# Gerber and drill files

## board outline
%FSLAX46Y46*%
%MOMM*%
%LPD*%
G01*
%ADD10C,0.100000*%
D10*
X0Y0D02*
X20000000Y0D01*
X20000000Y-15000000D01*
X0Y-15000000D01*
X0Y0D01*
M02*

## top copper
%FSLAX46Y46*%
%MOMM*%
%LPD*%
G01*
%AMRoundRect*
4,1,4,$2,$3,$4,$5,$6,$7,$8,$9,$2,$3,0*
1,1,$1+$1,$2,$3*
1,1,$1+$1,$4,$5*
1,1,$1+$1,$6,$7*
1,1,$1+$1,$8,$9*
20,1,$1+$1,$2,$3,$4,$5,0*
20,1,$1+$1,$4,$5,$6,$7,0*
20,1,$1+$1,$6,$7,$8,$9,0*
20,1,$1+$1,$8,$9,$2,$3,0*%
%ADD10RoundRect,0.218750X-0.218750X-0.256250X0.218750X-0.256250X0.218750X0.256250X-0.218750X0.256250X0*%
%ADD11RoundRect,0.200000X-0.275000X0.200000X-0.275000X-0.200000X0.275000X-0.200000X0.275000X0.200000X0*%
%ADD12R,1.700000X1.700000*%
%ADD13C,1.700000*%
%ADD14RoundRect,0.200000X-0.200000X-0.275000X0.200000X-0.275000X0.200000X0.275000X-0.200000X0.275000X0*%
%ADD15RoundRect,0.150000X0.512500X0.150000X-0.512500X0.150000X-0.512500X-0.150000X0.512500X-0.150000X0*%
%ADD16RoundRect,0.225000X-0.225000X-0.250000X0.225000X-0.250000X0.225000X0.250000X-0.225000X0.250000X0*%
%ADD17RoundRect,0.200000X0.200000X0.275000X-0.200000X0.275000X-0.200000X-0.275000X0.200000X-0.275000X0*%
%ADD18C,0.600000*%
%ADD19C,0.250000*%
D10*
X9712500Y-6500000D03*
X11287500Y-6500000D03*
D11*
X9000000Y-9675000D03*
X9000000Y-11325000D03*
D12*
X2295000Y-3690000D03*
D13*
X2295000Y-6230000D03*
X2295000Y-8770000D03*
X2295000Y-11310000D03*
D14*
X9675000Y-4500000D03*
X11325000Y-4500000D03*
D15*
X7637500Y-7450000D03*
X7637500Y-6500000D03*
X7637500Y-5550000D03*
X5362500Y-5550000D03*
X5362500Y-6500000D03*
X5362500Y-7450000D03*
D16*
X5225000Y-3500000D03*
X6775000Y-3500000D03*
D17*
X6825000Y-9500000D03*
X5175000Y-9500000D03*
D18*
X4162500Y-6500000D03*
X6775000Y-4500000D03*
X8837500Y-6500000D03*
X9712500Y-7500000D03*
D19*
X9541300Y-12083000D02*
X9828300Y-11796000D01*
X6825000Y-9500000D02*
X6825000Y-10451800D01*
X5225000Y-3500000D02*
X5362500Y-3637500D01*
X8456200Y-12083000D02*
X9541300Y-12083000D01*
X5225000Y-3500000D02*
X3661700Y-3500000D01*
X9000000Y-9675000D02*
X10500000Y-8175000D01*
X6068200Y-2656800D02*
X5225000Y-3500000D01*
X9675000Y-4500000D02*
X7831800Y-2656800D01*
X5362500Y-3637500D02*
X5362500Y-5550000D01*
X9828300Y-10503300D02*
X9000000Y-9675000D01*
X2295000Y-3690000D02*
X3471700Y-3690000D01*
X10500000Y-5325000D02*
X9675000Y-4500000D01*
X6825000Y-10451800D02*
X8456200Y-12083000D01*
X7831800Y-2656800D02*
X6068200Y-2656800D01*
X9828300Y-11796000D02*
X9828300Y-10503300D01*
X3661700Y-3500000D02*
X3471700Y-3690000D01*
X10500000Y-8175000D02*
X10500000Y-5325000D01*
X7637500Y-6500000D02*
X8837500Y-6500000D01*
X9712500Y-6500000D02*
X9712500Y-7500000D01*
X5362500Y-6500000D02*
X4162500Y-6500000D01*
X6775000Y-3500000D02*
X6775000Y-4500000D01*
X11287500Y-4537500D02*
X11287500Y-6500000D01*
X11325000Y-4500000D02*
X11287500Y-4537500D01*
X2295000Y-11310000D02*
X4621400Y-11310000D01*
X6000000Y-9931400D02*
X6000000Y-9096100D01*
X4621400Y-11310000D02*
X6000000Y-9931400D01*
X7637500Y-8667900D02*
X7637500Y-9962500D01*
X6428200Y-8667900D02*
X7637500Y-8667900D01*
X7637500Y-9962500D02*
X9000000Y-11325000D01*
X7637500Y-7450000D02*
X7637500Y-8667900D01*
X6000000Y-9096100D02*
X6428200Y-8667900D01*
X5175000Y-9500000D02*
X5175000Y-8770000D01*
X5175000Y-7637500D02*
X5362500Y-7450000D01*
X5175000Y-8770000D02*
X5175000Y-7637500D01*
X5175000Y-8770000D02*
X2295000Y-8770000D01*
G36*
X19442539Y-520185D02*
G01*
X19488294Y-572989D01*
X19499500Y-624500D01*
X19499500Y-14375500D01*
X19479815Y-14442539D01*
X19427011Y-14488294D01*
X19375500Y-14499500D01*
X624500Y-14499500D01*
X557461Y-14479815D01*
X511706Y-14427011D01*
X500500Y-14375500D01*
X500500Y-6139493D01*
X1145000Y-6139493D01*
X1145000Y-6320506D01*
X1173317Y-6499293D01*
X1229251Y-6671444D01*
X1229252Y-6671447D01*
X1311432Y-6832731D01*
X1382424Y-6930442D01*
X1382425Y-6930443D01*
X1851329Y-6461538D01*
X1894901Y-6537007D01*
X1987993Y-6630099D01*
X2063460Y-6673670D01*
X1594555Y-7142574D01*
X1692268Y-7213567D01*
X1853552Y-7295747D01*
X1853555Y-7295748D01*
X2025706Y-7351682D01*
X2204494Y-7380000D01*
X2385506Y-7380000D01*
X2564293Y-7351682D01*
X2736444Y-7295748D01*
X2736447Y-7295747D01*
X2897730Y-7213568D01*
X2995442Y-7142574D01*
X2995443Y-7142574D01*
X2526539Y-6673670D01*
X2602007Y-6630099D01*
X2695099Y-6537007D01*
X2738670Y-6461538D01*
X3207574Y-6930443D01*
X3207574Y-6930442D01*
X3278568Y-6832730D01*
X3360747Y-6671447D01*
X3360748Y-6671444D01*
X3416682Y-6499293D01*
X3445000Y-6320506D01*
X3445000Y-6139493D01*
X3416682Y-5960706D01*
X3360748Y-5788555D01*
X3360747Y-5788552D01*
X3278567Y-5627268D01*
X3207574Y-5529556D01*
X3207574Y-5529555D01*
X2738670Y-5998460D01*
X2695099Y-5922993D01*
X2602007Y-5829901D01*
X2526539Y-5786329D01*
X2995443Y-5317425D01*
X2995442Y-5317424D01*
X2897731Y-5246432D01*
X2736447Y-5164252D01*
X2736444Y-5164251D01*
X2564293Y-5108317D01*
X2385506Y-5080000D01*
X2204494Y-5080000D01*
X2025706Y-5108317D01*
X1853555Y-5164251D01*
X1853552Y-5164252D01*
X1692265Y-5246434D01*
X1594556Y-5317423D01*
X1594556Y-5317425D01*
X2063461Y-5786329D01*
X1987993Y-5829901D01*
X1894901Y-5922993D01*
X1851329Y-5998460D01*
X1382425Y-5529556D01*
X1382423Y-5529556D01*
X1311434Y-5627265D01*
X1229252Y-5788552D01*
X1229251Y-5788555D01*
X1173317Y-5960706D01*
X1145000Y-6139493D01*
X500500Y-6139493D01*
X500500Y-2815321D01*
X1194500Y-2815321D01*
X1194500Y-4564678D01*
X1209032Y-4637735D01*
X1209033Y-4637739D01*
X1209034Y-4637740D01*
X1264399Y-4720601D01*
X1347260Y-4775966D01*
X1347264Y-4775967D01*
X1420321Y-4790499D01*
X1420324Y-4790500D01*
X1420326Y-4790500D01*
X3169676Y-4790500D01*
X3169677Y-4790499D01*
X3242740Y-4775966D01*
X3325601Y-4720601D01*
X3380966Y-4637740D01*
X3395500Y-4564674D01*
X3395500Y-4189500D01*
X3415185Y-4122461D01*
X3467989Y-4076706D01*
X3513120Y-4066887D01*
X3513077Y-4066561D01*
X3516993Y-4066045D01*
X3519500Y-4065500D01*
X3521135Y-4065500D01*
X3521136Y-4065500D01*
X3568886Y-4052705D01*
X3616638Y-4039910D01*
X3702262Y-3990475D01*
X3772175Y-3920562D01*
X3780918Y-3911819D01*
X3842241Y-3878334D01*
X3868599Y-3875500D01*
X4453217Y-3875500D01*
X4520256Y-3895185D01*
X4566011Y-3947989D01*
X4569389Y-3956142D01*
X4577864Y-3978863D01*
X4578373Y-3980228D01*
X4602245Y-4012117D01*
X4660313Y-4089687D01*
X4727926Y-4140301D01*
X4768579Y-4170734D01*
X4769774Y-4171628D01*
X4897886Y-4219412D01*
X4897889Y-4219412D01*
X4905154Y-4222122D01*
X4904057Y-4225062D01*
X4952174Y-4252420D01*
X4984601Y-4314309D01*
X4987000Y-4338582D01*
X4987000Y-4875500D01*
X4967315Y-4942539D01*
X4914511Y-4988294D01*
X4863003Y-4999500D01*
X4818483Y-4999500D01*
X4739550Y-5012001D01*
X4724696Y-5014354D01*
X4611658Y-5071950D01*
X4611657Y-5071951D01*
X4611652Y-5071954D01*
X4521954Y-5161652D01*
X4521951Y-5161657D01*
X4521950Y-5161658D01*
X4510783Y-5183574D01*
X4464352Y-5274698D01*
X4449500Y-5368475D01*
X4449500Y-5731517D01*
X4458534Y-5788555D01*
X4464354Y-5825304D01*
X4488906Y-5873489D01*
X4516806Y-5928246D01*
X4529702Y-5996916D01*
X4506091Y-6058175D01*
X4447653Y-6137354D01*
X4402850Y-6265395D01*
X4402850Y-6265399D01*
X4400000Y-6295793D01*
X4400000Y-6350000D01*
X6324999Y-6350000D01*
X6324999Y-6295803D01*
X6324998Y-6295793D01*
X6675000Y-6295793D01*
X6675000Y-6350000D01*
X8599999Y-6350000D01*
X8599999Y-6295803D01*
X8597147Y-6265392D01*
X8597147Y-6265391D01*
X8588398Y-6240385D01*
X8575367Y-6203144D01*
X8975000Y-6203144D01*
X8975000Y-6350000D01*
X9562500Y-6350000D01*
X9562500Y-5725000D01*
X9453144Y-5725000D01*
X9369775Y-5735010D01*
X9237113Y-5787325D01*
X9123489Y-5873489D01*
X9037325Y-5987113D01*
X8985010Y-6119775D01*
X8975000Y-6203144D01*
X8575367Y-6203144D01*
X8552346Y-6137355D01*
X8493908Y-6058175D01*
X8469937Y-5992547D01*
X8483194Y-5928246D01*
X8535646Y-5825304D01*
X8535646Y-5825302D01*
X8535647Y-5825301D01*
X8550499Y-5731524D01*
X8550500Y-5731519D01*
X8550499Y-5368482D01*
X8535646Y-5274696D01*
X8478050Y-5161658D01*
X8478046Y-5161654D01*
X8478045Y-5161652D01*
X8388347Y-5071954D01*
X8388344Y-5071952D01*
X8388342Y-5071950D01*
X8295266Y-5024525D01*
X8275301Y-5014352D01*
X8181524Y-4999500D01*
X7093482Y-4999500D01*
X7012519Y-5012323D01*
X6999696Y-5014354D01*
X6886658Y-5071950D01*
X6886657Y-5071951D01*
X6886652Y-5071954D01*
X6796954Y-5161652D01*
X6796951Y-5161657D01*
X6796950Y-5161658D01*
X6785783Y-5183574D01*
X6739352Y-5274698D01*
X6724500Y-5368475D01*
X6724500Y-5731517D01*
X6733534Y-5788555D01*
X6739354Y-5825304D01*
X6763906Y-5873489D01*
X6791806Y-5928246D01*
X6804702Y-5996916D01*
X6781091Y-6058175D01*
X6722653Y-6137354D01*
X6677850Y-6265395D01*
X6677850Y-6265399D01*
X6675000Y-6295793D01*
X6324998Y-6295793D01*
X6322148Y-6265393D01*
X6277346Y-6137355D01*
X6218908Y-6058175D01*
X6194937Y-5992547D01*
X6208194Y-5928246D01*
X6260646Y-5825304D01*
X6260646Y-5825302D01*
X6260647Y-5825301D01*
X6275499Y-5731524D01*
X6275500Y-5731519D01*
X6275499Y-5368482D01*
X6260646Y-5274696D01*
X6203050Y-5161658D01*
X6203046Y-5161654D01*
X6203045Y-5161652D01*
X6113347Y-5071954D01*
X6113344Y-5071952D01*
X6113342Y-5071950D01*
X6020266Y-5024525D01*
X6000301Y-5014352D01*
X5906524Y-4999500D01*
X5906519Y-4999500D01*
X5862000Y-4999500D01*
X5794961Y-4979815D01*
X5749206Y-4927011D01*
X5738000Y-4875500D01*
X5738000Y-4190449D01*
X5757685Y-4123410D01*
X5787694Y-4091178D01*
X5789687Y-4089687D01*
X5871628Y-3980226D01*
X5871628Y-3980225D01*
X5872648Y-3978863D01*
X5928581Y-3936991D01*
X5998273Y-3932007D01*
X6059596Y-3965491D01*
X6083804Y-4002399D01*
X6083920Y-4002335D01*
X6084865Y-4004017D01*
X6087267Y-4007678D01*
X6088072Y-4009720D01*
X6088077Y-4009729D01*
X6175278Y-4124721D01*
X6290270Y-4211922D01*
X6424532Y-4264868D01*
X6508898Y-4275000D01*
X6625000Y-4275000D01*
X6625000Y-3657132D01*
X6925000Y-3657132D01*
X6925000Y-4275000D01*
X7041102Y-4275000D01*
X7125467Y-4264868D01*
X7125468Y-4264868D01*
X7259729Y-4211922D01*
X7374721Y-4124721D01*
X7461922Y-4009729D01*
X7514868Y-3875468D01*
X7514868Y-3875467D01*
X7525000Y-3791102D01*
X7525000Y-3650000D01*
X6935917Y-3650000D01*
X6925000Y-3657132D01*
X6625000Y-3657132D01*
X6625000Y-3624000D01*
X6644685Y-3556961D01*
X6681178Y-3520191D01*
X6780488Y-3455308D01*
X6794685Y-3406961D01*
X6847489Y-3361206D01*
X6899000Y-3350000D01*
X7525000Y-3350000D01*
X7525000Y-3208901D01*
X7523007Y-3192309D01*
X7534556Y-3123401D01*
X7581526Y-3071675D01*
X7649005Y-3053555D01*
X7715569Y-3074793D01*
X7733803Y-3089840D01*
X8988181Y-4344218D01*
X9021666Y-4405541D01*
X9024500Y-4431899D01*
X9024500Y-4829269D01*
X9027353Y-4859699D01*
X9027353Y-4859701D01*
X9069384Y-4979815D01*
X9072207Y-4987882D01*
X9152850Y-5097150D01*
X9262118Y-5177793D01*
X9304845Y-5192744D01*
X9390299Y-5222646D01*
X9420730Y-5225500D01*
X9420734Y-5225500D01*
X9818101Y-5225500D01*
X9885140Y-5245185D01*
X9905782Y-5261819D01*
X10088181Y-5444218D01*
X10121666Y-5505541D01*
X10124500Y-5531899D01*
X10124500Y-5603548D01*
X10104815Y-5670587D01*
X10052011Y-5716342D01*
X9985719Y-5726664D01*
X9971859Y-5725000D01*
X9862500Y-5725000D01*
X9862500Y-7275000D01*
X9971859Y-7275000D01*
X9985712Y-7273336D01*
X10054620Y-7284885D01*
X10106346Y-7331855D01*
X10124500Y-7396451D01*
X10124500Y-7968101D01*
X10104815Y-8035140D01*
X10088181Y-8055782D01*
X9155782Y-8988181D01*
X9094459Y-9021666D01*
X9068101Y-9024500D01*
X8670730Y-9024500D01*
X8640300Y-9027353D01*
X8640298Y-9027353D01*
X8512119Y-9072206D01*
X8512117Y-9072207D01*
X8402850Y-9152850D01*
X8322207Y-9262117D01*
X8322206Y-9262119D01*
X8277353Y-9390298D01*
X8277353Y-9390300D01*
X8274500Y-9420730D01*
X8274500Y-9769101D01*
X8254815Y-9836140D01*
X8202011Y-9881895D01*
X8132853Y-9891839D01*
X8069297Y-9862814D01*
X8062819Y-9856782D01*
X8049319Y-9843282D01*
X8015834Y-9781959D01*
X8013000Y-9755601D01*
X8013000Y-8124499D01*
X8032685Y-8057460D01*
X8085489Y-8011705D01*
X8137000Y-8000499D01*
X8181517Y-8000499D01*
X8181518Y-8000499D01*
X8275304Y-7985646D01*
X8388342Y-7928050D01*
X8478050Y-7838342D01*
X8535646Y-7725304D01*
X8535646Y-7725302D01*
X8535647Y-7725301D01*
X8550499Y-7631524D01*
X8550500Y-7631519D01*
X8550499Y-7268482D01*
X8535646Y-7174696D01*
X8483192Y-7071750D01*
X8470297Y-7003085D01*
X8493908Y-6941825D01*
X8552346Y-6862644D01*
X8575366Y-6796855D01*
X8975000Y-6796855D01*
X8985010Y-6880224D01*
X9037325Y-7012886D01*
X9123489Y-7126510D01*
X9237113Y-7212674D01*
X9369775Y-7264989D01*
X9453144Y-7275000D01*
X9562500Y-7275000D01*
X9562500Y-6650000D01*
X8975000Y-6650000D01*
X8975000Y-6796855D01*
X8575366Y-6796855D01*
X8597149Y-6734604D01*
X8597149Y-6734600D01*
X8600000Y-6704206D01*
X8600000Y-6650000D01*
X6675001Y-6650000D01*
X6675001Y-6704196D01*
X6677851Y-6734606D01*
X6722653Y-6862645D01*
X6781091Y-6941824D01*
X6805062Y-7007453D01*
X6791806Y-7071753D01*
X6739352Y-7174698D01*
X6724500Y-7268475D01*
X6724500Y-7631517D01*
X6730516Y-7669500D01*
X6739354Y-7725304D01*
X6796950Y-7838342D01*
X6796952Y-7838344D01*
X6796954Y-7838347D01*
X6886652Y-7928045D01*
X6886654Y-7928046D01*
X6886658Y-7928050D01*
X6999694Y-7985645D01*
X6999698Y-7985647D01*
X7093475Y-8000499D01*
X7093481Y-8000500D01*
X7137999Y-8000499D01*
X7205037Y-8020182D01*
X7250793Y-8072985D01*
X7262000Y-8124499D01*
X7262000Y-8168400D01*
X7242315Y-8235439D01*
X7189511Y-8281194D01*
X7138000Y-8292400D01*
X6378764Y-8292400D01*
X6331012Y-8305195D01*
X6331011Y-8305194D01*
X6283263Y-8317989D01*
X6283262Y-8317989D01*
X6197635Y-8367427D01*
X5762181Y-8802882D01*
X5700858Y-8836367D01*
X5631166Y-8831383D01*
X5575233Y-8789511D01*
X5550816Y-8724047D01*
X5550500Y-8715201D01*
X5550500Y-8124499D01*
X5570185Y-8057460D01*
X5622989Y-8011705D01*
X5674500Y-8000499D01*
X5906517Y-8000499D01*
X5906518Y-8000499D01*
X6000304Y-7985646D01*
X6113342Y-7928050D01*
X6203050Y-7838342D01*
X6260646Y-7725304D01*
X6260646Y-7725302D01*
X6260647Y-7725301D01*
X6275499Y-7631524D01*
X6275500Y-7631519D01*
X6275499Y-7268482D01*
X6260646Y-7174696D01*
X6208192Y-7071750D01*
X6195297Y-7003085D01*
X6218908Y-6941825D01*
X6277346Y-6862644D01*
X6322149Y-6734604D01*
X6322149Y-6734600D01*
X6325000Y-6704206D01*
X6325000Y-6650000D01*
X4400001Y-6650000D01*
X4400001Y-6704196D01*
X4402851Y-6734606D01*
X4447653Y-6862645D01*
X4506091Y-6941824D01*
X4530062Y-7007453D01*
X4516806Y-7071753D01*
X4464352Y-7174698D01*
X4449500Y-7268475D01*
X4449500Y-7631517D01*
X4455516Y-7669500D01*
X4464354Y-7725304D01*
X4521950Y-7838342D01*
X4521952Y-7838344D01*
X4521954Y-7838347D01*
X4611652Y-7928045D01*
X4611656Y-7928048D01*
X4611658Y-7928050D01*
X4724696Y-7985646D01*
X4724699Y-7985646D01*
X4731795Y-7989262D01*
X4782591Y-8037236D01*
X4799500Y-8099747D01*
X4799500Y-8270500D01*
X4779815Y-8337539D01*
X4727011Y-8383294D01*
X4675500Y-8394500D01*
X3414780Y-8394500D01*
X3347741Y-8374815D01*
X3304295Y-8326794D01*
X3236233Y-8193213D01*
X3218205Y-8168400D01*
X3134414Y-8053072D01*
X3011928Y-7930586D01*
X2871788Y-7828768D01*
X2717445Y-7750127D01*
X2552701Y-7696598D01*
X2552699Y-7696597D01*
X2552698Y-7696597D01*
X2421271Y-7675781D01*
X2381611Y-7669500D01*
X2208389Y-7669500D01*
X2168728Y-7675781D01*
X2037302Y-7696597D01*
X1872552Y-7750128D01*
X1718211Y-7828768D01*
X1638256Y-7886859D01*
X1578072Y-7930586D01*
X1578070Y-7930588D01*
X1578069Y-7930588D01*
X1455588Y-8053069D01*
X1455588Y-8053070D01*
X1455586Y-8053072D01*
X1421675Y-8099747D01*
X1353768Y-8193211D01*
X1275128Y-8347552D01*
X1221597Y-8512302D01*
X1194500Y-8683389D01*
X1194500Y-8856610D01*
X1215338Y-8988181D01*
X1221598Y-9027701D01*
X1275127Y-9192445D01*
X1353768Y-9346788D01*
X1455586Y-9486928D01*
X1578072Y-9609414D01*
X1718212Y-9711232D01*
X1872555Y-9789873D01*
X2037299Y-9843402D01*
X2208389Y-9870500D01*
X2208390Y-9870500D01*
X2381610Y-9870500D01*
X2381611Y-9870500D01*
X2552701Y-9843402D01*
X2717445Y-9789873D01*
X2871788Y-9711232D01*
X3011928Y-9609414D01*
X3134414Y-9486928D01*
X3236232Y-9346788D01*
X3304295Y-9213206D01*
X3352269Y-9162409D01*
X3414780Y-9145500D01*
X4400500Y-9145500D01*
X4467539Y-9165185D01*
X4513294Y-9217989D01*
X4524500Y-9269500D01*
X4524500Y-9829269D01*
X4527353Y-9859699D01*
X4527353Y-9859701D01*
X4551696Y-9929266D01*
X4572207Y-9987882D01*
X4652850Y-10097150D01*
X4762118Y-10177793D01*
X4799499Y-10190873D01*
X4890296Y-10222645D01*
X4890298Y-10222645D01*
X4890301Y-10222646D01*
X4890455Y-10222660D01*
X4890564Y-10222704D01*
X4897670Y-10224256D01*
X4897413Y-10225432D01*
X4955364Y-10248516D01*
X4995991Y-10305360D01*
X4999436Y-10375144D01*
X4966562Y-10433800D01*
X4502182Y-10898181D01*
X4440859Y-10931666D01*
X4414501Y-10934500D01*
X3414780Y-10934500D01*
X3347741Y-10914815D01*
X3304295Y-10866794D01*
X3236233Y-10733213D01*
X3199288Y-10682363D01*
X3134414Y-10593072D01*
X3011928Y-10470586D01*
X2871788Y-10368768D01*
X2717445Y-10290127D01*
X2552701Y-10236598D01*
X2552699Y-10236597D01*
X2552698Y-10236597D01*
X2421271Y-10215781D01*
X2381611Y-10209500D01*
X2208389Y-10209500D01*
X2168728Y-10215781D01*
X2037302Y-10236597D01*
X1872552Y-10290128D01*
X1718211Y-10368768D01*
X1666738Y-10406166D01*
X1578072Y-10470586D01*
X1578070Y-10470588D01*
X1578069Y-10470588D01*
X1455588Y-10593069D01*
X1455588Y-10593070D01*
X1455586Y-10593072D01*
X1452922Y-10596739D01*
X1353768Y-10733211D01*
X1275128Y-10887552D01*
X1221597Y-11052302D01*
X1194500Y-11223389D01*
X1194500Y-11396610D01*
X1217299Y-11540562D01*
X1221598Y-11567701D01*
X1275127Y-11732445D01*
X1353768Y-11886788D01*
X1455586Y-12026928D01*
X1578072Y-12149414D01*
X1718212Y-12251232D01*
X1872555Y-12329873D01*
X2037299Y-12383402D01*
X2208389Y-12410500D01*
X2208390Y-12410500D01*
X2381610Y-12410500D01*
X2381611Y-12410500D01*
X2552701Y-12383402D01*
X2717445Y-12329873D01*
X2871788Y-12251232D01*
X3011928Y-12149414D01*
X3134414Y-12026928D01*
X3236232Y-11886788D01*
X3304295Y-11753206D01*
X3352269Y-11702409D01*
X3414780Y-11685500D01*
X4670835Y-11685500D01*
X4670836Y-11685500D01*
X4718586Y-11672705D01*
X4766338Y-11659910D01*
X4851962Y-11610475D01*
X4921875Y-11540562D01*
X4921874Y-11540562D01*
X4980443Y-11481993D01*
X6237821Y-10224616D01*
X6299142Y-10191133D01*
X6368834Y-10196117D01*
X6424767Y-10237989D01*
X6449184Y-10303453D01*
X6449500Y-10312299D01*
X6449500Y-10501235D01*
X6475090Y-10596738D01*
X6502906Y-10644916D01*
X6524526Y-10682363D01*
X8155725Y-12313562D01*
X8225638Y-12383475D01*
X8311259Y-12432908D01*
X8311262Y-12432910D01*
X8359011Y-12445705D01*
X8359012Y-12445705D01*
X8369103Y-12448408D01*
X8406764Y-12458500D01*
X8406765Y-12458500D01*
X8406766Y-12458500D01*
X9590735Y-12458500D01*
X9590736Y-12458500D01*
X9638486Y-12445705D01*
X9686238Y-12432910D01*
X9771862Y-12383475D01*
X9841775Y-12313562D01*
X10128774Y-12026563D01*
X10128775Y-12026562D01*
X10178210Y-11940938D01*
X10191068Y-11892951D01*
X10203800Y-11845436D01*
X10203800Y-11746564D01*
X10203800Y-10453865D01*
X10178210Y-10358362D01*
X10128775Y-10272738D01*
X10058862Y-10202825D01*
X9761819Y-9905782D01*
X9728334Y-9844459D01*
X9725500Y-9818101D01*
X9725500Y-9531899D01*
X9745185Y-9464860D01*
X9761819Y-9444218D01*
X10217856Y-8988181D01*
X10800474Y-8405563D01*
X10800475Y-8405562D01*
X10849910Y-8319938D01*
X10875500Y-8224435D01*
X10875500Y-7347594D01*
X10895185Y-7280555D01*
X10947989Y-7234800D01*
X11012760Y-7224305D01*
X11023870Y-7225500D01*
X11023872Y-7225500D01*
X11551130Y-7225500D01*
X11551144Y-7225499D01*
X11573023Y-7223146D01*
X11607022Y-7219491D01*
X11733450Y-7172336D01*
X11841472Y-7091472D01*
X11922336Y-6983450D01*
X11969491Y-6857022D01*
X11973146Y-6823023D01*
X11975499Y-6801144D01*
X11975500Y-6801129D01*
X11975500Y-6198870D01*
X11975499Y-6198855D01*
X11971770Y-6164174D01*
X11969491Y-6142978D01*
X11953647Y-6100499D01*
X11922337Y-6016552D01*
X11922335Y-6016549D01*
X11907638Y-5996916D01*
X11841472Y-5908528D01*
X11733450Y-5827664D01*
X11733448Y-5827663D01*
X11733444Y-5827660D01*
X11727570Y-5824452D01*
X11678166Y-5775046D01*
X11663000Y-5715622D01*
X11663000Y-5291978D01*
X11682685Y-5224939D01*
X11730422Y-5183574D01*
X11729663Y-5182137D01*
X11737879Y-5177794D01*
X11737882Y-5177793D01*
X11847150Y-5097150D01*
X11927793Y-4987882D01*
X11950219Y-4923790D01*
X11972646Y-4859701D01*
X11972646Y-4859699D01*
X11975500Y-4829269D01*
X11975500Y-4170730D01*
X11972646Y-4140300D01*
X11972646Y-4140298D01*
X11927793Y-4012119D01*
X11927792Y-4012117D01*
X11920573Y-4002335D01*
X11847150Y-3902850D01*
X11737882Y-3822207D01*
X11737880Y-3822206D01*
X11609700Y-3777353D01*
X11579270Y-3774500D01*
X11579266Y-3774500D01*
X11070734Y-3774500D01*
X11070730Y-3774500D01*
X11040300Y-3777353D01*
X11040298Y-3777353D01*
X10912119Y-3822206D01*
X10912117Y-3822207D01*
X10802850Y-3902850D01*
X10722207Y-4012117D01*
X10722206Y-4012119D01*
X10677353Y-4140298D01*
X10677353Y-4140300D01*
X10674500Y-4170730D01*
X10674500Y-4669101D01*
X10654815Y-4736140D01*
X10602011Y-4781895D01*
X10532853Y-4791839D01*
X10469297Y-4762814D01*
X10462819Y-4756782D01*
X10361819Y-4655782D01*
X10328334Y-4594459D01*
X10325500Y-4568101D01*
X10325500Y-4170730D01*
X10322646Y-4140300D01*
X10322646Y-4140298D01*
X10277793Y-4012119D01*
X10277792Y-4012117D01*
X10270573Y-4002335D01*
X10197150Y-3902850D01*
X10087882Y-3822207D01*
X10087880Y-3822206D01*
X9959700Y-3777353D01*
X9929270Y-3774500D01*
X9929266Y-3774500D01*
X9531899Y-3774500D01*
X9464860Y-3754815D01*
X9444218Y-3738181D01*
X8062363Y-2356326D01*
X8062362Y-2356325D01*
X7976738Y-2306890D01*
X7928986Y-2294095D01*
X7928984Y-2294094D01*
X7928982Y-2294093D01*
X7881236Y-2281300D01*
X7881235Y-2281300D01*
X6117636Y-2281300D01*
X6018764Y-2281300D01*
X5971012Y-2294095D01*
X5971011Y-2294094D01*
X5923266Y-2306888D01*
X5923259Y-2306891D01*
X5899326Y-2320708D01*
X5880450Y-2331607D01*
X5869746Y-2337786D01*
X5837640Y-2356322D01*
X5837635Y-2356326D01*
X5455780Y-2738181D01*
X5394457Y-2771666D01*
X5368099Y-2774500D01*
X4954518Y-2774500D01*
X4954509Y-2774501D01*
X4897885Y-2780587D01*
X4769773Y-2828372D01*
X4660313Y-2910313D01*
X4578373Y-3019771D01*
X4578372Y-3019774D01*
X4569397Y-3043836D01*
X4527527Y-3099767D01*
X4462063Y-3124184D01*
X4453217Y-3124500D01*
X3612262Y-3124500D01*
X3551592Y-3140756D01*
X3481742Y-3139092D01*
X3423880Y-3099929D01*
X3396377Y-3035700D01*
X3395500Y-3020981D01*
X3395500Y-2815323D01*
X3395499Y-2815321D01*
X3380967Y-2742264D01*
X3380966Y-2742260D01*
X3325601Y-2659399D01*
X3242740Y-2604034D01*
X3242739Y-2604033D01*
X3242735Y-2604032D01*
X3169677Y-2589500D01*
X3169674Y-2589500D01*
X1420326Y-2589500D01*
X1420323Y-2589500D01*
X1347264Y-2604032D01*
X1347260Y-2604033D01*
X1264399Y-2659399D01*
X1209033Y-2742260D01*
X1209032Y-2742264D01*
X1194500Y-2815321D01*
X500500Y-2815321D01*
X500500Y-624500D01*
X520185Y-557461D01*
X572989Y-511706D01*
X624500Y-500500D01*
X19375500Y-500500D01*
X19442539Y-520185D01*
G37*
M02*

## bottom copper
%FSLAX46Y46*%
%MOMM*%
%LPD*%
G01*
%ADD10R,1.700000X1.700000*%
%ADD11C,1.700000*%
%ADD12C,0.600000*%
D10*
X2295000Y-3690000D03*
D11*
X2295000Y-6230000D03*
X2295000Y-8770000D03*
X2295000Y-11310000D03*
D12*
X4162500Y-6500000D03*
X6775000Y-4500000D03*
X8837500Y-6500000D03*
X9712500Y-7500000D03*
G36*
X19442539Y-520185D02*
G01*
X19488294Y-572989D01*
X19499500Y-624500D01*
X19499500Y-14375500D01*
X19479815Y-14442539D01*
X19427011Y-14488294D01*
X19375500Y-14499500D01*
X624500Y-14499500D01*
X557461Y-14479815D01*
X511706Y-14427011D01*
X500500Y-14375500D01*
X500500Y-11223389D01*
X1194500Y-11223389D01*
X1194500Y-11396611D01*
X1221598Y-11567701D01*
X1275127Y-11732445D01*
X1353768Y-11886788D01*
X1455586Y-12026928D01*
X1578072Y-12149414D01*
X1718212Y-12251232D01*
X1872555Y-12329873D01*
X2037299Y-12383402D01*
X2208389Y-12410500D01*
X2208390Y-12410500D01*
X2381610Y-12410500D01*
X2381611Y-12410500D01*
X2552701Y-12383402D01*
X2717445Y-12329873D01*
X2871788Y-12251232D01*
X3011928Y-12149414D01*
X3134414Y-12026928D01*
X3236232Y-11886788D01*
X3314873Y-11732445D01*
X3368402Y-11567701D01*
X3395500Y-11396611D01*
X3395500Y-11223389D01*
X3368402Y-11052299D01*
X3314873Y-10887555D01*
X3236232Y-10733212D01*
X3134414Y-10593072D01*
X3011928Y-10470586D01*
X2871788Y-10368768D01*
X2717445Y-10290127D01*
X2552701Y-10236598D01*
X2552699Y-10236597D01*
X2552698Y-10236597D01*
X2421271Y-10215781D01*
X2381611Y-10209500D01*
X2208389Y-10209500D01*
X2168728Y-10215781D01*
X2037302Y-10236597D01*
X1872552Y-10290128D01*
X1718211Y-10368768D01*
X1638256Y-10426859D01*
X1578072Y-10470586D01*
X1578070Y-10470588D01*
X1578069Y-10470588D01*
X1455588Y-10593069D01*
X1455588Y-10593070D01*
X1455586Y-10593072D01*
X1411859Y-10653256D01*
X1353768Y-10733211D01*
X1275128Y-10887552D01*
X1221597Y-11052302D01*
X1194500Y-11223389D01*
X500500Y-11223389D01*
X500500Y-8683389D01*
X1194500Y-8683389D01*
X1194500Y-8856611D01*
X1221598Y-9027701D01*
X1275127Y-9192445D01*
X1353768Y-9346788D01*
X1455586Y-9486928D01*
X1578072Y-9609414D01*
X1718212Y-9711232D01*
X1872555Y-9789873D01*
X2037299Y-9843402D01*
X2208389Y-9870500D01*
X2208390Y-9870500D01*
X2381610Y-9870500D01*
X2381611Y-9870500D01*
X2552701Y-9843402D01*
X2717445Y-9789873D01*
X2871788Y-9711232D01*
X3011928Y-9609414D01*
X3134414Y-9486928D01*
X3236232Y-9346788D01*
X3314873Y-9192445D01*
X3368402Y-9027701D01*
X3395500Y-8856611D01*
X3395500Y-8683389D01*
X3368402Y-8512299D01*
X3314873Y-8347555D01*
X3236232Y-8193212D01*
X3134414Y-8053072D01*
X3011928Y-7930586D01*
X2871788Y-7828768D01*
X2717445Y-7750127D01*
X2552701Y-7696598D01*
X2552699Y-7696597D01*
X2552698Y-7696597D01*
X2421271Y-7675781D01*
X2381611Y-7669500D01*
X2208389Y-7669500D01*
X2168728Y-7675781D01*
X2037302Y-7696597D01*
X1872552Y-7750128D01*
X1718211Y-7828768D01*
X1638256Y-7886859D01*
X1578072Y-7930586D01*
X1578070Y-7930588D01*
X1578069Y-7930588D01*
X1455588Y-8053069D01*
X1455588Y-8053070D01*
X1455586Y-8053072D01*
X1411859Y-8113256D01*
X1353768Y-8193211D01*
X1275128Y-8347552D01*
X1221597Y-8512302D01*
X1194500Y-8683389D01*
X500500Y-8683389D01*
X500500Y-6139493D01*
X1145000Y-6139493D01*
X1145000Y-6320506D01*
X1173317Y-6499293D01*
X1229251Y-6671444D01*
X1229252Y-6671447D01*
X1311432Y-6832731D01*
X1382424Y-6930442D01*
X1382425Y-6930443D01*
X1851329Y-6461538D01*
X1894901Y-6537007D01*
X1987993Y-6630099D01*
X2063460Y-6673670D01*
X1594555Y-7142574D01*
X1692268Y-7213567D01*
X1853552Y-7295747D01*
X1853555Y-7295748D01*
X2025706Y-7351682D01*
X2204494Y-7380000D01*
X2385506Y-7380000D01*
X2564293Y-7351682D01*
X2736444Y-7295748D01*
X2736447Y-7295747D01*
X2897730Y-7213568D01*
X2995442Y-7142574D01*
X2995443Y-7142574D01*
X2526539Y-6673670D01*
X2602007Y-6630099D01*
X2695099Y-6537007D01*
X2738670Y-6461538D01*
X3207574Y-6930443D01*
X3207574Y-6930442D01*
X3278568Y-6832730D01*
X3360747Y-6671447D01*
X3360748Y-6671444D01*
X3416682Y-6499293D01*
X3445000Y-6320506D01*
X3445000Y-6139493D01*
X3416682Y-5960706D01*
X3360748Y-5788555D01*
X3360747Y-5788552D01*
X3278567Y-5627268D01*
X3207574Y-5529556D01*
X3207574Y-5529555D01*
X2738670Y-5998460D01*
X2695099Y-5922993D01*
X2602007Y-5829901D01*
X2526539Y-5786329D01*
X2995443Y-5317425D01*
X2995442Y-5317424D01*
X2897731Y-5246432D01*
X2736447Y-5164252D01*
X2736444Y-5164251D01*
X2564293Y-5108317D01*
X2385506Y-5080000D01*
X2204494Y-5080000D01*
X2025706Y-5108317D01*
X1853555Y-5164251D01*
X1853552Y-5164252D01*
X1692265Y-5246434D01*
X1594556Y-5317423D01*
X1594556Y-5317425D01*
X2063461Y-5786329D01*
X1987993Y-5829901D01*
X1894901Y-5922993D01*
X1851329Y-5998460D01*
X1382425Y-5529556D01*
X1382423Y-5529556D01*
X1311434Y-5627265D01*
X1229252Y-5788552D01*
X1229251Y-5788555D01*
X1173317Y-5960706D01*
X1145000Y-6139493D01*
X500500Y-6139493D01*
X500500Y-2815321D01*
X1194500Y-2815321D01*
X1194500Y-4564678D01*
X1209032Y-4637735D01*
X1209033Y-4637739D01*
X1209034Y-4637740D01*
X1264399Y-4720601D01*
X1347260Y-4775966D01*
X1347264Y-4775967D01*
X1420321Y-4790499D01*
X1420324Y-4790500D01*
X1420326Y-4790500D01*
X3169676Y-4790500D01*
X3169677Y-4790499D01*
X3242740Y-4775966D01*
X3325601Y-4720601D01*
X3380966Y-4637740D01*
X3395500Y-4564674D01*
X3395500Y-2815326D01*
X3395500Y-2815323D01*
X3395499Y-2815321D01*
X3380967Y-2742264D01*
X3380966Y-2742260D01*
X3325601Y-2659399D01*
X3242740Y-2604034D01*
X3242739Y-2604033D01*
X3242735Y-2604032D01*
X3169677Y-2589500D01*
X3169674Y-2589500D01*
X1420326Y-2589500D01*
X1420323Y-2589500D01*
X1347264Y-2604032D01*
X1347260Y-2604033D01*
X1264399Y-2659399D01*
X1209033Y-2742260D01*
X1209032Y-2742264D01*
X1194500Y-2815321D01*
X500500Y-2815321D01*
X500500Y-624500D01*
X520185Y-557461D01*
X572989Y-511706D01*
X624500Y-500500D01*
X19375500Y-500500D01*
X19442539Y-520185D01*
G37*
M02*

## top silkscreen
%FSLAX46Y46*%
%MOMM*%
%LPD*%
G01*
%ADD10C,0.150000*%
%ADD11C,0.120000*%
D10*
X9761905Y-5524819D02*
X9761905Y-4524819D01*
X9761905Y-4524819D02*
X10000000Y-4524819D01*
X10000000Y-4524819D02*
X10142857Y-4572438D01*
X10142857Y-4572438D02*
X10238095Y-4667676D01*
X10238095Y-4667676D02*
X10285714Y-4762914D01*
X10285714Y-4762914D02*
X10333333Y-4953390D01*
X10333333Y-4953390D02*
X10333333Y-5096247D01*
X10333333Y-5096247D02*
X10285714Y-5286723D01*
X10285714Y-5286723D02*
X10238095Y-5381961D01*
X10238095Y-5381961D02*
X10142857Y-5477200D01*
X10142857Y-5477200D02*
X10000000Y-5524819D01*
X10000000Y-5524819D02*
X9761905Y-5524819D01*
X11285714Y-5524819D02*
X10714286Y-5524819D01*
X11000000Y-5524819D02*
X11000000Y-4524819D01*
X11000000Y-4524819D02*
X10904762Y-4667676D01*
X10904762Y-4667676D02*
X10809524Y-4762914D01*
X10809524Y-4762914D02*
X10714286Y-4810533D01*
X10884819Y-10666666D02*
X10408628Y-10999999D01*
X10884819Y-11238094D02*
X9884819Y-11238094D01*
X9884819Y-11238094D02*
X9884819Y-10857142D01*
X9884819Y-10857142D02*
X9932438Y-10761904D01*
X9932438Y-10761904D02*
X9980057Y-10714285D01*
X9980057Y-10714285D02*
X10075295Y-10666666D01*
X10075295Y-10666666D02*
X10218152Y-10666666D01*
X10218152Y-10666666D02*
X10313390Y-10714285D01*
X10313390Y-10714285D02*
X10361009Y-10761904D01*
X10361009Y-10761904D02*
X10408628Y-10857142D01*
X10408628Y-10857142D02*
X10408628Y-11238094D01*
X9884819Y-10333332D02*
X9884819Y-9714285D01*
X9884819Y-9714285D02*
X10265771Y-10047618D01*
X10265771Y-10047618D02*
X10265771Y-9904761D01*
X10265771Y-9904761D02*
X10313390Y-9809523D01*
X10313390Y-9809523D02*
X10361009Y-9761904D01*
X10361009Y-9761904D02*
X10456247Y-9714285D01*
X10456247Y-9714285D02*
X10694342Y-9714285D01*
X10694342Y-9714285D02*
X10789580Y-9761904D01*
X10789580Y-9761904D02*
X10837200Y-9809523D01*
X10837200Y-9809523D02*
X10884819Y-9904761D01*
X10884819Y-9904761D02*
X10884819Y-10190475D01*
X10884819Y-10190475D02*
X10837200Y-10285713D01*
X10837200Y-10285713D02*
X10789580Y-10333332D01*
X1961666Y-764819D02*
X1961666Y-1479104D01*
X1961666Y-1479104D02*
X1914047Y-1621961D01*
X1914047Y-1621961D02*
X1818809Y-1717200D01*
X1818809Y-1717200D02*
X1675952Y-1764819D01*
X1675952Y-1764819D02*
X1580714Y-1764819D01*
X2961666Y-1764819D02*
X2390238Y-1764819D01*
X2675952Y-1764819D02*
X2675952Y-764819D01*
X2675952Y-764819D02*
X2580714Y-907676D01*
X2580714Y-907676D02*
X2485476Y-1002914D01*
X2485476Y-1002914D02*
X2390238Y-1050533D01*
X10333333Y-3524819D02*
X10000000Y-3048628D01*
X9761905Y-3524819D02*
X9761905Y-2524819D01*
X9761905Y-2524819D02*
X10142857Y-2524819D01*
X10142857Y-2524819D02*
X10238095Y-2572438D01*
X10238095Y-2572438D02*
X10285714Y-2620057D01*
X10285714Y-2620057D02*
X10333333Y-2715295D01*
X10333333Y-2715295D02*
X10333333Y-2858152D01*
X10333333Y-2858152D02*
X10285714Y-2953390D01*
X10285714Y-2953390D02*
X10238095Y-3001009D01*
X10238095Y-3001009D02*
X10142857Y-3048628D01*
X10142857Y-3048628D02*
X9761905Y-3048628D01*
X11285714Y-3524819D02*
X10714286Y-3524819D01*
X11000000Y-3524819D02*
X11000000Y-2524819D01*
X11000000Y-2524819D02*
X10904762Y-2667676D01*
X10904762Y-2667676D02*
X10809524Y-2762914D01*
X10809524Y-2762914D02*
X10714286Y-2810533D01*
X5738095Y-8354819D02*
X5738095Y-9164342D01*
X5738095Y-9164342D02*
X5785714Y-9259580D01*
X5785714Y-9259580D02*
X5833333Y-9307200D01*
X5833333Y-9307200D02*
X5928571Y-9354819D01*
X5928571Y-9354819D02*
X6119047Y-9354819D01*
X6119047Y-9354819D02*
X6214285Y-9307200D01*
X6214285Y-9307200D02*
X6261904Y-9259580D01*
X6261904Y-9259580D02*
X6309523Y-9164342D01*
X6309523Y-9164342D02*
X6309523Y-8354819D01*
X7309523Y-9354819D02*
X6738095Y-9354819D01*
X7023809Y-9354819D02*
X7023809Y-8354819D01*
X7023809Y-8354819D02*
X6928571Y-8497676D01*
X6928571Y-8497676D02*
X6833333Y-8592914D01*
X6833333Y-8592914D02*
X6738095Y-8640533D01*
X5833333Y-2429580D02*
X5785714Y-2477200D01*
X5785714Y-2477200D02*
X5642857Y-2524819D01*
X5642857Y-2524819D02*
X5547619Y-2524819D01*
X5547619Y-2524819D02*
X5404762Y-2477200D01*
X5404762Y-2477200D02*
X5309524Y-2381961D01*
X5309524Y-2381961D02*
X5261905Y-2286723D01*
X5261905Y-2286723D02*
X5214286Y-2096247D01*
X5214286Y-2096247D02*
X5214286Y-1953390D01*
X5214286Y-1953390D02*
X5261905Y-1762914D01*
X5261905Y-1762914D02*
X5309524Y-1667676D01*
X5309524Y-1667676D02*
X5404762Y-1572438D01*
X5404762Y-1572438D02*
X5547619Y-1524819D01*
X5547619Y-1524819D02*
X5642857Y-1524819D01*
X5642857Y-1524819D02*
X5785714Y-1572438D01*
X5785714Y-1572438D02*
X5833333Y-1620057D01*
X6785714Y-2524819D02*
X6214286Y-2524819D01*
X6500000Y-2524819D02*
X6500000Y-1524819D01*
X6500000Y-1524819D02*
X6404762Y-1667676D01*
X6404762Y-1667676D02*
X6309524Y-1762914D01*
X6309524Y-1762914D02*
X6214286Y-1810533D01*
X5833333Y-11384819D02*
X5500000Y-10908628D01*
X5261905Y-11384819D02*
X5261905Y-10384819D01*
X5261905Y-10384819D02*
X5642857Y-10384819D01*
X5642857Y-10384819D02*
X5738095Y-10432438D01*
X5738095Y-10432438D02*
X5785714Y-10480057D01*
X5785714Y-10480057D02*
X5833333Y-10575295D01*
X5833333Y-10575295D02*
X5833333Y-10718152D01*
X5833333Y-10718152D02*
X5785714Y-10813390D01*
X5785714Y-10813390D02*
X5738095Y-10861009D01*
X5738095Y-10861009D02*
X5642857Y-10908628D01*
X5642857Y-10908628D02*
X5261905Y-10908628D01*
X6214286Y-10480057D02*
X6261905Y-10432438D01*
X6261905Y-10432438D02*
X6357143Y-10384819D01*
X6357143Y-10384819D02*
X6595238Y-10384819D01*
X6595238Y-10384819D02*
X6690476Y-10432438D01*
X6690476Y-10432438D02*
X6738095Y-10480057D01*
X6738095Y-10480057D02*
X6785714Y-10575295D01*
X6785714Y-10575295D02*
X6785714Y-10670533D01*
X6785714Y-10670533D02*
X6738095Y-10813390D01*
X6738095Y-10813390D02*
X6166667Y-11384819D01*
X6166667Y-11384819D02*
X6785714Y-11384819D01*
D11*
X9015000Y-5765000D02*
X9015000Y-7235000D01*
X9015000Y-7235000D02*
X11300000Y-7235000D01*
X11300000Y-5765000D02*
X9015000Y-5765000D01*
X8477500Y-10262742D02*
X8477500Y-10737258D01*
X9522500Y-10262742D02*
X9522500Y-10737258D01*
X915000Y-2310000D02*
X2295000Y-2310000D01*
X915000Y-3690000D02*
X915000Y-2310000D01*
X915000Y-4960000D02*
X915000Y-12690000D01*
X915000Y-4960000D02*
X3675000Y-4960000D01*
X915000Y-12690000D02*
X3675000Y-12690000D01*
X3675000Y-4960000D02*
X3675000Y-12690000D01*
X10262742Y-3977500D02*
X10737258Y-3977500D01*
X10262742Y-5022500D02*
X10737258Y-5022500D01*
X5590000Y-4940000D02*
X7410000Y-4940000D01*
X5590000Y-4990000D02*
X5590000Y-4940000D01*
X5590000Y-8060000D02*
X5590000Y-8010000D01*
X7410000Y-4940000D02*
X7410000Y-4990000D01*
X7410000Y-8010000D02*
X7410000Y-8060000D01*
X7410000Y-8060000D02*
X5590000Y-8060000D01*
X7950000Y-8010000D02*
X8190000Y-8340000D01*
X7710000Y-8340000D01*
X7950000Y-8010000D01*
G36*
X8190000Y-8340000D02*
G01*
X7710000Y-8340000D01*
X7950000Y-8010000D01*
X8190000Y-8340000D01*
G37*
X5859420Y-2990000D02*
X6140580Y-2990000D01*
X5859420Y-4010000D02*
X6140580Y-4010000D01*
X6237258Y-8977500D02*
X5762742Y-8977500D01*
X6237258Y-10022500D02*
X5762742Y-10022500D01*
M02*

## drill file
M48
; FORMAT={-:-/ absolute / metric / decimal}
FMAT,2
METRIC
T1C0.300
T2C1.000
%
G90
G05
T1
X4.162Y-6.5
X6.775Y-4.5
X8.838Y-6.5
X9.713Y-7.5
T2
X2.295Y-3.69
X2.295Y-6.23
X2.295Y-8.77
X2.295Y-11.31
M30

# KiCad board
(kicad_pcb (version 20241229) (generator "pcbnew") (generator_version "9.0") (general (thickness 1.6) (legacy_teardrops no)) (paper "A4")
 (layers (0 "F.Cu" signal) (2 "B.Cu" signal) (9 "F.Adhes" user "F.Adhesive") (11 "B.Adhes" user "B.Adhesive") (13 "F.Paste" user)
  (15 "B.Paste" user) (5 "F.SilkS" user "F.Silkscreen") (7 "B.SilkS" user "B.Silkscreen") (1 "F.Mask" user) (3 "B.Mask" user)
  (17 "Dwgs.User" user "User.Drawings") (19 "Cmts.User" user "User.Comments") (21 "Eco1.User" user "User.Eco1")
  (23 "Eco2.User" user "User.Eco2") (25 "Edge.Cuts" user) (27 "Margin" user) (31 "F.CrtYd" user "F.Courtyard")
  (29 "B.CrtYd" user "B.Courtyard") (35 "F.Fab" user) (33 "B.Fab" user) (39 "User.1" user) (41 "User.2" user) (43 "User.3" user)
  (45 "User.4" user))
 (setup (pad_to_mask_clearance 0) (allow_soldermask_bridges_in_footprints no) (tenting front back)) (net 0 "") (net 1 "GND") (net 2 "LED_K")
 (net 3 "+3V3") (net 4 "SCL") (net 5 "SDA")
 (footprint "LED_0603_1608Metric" (layer "F.Cu") (at 10.5 6.5)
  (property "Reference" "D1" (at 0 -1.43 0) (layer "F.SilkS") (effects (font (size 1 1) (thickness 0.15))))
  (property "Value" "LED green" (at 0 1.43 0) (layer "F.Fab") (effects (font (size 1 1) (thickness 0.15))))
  (fp_line (start -1.485 -0.735) (end -1.485 0.735) (stroke (width 0.12) (type solid)) (layer "F.SilkS"))
  (fp_line (start -1.485 0.735) (end 0.8 0.735) (stroke (width 0.12) (type solid)) (layer "F.SilkS"))
  (fp_line (start 0.8 -0.735) (end -1.485 -0.735) (stroke (width 0.12) (type solid)) (layer "F.SilkS"))
  (pad "1" smd roundrect (at -0.7875 0) (size 0.875 0.95) (layers "F.Cu" "F.Mask" "F.Paste") (roundrect_rratio 0.25) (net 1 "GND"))
  (pad "2" smd roundrect (at 0.7875 0) (size 0.875 0.95) (layers "F.Cu" "F.Mask" "F.Paste") (roundrect_rratio 0.25) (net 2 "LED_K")))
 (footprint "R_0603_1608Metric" (layer "F.Cu") (at 9 10.5 -90)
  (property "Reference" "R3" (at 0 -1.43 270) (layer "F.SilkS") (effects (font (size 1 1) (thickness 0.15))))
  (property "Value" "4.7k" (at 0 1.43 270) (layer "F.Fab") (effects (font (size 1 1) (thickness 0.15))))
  (fp_line (start -0.237258 0.5225) (end 0.237258 0.5225) (stroke (width 0.12) (type solid)) (layer "F.SilkS"))
  (fp_line (start -0.237258 -0.5225) (end 0.237258 -0.5225) (stroke (width 0.12) (type solid)) (layer "F.SilkS"))
  (pad "1" smd roundrect (at -0.825 0 270) (size 0.8 0.95) (layers "F.Cu" "F.Mask" "F.Paste") (roundrect_rratio 0.25) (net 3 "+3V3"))
  (pad "2" smd roundrect (at 0.825 0 270) (size 0.8 0.95) (layers "F.Cu" "F.Mask" "F.Paste") (roundrect_rratio 0.25) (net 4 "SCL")))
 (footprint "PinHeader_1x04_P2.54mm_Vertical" (layer "F.Cu") (at 2.295 3.69)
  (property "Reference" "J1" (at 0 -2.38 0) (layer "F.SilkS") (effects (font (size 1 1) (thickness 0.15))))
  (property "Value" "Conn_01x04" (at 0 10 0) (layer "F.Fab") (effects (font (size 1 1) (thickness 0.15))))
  (fp_line (start -1.38 -1.38) (end 0 -1.38) (stroke (width 0.12) (type solid)) (layer "F.SilkS"))
  (fp_line (start -1.38 0) (end -1.38 -1.38) (stroke (width 0.12) (type solid)) (layer "F.SilkS"))
  (fp_line (start -1.38 1.27) (end -1.38 9) (stroke (width 0.12) (type solid)) (layer "F.SilkS"))
  (fp_line (start -1.38 1.27) (end 1.38 1.27) (stroke (width 0.12) (type solid)) (layer "F.SilkS"))
  (fp_line (start -1.38 9) (end 1.38 9) (stroke (width 0.12) (type solid)) (layer "F.SilkS"))
  (fp_line (start 1.38 1.27) (end 1.38 9) (stroke (width 0.12) (type solid)) (layer "F.SilkS"))
  (pad "1" thru_hole rect (at 0 0) (size 1.7 1.7) (drill 1) (layers "*.Cu" "*.Mask") (remove_unused_layers no) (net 3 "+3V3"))
  (pad "2" thru_hole circle (at 0 2.54) (size 1.7 1.7) (drill 1) (layers "*.Cu" "*.Mask") (remove_unused_layers no) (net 1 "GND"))
  (pad "3" thru_hole circle (at 0 5.08) (size 1.7 1.7) (drill 1) (layers "*.Cu" "*.Mask") (remove_unused_layers no) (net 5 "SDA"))
  (pad "4" thru_hole circle (at 0 7.62) (size 1.7 1.7) (drill 1) (layers "*.Cu" "*.Mask") (remove_unused_layers no) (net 4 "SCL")))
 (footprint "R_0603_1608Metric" (layer "F.Cu") (at 10.5 4.5)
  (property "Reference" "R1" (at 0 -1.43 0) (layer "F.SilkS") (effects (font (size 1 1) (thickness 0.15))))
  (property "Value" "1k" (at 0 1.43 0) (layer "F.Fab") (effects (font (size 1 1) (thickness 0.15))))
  (fp_line (start -0.237258 -0.5225) (end 0.237258 -0.5225) (stroke (width 0.12) (type solid)) (layer "F.SilkS"))
  (fp_line (start -0.237258 0.5225) (end 0.237258 0.5225) (stroke (width 0.12) (type solid)) (layer "F.SilkS"))
  (pad "1" smd roundrect (at -0.825 0) (size 0.8 0.95) (layers "F.Cu" "F.Mask" "F.Paste") (roundrect_rratio 0.25) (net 3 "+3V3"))
  (pad "2" smd roundrect (at 0.825 0) (size 0.8 0.95) (layers "F.Cu" "F.Mask" "F.Paste") (roundrect_rratio 0.25) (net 2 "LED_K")))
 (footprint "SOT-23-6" (layer "F.Cu") (at 6.5 6.5 180)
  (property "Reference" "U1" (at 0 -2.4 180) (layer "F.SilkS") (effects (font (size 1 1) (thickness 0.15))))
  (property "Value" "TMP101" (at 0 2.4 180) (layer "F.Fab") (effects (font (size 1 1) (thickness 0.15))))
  (fp_line (start 0.91 1.56) (end -0.91 1.56) (stroke (width 0.12) (type solid)) (layer "F.SilkS"))
  (fp_line (start 0.91 1.51) (end 0.91 1.56) (stroke (width 0.12) (type solid)) (layer "F.SilkS"))
  (fp_line (start 0.91 -1.56) (end 0.91 -1.51) (stroke (width 0.12) (type solid)) (layer "F.SilkS"))
  (fp_line (start -0.91 1.56) (end -0.91 1.51) (stroke (width 0.12) (type solid)) (layer "F.SilkS"))
  (fp_line (start -0.91 -1.51) (end -0.91 -1.56) (stroke (width 0.12) (type solid)) (layer "F.SilkS"))
  (fp_line (start -0.91 -1.56) (end 0.91 -1.56) (stroke (width 0.12) (type solid)) (layer "F.SilkS"))
  (fp_poly (pts (xy -1.45 -1.51) (xy -1.69 -1.84) (xy -1.21 -1.84)) (stroke (width 0.12) (type solid)) (fill yes) (layer "F.SilkS"))
  (pad "1" smd roundrect (at -1.1375 -0.95 180) (size 1.325 0.6) (layers "F.Cu" "F.Mask" "F.Paste") (roundrect_rratio 0.25) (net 4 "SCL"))
  (pad "2" smd roundrect (at -1.1375 0 180) (size 1.325 0.6) (layers "F.Cu" "F.Mask" "F.Paste") (roundrect_rratio 0.25) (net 1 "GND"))
  (pad "3" smd roundrect (at -1.1375 0.95 180) (size 1.325 0.6) (layers "F.Cu" "F.Mask" "F.Paste") (roundrect_rratio 0.25))
  (pad "4" smd roundrect (at 1.1375 0.95 180) (size 1.325 0.6) (layers "F.Cu" "F.Mask" "F.Paste") (roundrect_rratio 0.25) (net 3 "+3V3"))
  (pad "5" smd roundrect (at 1.1375 0 180) (size 1.325 0.6) (layers "F.Cu" "F.Mask" "F.Paste") (roundrect_rratio 0.25) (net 1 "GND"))
  (pad "6" smd roundrect (at 1.1375 -0.95 180) (size 1.325 0.6) (layers "F.Cu" "F.Mask" "F.Paste") (roundrect_rratio 0.25) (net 5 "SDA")))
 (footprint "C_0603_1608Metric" (layer "F.Cu") (at 6 3.5)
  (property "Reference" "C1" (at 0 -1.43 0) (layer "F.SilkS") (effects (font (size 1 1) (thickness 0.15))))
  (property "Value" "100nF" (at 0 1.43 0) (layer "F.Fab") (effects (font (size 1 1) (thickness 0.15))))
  (fp_line (start -0.14058 -0.51) (end 0.14058 -0.51) (stroke (width 0.12) (type solid)) (layer "F.SilkS"))
  (fp_line (start -0.14058 0.51) (end 0.14058 0.51) (stroke (width 0.12) (type solid)) (layer "F.SilkS"))
  (pad "1" smd roundrect (at -0.775 0) (size 0.9 0.95) (layers "F.Cu" "F.Mask" "F.Paste") (roundrect_rratio 0.25) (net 3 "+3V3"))
  (pad "2" smd roundrect (at 0.775 0) (size 0.9 0.95) (layers "F.Cu" "F.Mask" "F.Paste") (roundrect_rratio 0.25) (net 1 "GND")))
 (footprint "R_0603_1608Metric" (layer "F.Cu") (at 6 9.5 180)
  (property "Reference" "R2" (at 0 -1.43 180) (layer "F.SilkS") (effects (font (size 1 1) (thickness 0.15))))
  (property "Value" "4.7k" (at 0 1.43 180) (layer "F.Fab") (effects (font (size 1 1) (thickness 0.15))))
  (fp_line (start -0.237258 0.5225) (end 0.237258 0.5225) (stroke (width 0.12) (type solid)) (layer "F.SilkS"))
  (fp_line (start -0.237258 -0.5225) (end 0.237258 -0.5225) (stroke (width 0.12) (type solid)) (layer "F.SilkS"))
  (pad "1" smd roundrect (at -0.825 0 180) (size 0.8 0.95) (layers "F.Cu" "F.Mask" "F.Paste") (roundrect_rratio 0.25) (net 3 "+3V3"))
  (pad "2" smd roundrect (at 0.825 0 180) (size 0.8 0.95) (layers "F.Cu" "F.Mask" "F.Paste") (roundrect_rratio 0.25) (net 5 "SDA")))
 (gr_rect (start 0 0) (end 20 15) (stroke (width 0.1) (type default)) (fill no) (layer "Edge.Cuts"))
 (segment (start 9.5413 12.083) (end 9.8283 11.796) (width 0.25) (layer "F.Cu") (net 3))
 (segment (start 6.825 9.5) (end 6.825 10.4518) (width 0.25) (layer "F.Cu") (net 3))
 (segment (start 5.225 3.5) (end 5.3625 3.6375) (width 0.25) (layer "F.Cu") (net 3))
 (segment (start 8.4562 12.083) (end 9.5413 12.083) (width 0.25) (layer "F.Cu") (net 3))
 (segment (start 5.225 3.5) (end 3.6617 3.5) (width 0.25) (layer "F.Cu") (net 3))
 (segment (start 9 9.675) (end 10.5 8.175) (width 0.25) (layer "F.Cu") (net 3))
 (segment (start 6.0682 2.6568) (end 5.225 3.5) (width 0.25) (layer "F.Cu") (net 3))
 (segment (start 9.675 4.5) (end 7.8318 2.6568) (width 0.25) (layer "F.Cu") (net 3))
 (segment (start 5.3625 3.6375) (end 5.3625 5.55) (width 0.25) (layer "F.Cu") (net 3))
 (segment (start 9.8283 10.5033) (end 9 9.675) (width 0.25) (layer "F.Cu") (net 3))
 (segment (start 2.295 3.69) (end 3.4717 3.69) (width 0.25) (layer "F.Cu") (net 3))
 (segment (start 10.5 5.325) (end 9.675 4.5) (width 0.25) (layer "F.Cu") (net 3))
 (segment (start 6.825 10.4518) (end 8.4562 12.083) (width 0.25) (layer "F.Cu") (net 3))
 (segment (start 7.8318 2.6568) (end 6.0682 2.6568) (width 0.25) (layer "F.Cu") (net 3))
 (segment (start 9.8283 11.796) (end 9.8283 10.5033) (width 0.25) (layer "F.Cu") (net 3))
 (segment (start 3.6617 3.5) (end 3.4717 3.69) (width 0.25) (layer "F.Cu") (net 3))
 (segment (start 10.5 8.175) (end 10.5 5.325) (width 0.25) (layer "F.Cu") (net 3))
 (segment (start 7.6375 6.5) (end 8.8375 6.5) (width 0.25) (layer "F.Cu") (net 1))
 (segment (start 9.7125 6.5) (end 9.7125 7.5) (width 0.25) (layer "F.Cu") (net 1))
 (segment (start 5.3625 6.5) (end 4.1625 6.5) (width 0.25) (layer "F.Cu") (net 1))
 (segment (start 6.775 3.5) (end 6.775 4.5) (width 0.25) (layer "F.Cu") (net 1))
 (via (at 4.1625 6.5) (size 0.6) (drill 0.3) (layers "F.Cu" "B.Cu") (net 1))
 (via (at 6.775 4.5) (size 0.6) (drill 0.3) (layers "F.Cu" "B.Cu") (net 1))
 (via (at 8.8375 6.5) (size 0.6) (drill 0.3) (layers "F.Cu" "B.Cu") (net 1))
 (via (at 9.7125 7.5) (size 0.6) (drill 0.3) (layers "F.Cu" "B.Cu") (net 1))
 (segment (start 11.2875 4.5375) (end 11.2875 6.5) (width 0.25) (layer "F.Cu") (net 2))
 (segment (start 11.325 4.5) (end 11.2875 4.5375) (width 0.25) (layer "F.Cu") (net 2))
 (segment (start 2.295 11.31) (end 4.6214 11.31) (width 0.25) (layer "F.Cu") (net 4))
 (segment (start 6 9.9314) (end 6 9.0961) (width 0.25) (layer "F.Cu") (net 4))
 (segment (start 4.6214 11.31) (end 6 9.9314) (width 0.25) (layer "F.Cu") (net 4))
 (segment (start 7.6375 8.6679) (end 7.6375 9.9625) (width 0.25) (layer "F.Cu") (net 4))
 (segment (start 6.4282 8.6679) (end 7.6375 8.6679) (width 0.25) (layer "F.Cu") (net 4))
 (segment (start 7.6375 9.9625) (end 9 11.325) (width 0.25) (layer "F.Cu") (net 4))
 (segment (start 7.6375 7.45) (end 7.6375 8.6679) (width 0.25) (layer "F.Cu") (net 4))
 (segment (start 6 9.0961) (end 6.4282 8.6679) (width 0.25) (layer "F.Cu") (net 4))
 (segment (start 5.175 9.5) (end 5.175 8.77) (width 0.25) (layer "F.Cu") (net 5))
 (segment (start 5.175 7.6375) (end 5.3625 7.45) (width 0.25) (layer "F.Cu") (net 5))
 (segment (start 5.175 8.77) (end 5.175 7.6375) (width 0.25) (layer "F.Cu") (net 5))
 (segment (start 5.175 8.77) (end 2.295 8.77) (width 0.25) (layer "F.Cu") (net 5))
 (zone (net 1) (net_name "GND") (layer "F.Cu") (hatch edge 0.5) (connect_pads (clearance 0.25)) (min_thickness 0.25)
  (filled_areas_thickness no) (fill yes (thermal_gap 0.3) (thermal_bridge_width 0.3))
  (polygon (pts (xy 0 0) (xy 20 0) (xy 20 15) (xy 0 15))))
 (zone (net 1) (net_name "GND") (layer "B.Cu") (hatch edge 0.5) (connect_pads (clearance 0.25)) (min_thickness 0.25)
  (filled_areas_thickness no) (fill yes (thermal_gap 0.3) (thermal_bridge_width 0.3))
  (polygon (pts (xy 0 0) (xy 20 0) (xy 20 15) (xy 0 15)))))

